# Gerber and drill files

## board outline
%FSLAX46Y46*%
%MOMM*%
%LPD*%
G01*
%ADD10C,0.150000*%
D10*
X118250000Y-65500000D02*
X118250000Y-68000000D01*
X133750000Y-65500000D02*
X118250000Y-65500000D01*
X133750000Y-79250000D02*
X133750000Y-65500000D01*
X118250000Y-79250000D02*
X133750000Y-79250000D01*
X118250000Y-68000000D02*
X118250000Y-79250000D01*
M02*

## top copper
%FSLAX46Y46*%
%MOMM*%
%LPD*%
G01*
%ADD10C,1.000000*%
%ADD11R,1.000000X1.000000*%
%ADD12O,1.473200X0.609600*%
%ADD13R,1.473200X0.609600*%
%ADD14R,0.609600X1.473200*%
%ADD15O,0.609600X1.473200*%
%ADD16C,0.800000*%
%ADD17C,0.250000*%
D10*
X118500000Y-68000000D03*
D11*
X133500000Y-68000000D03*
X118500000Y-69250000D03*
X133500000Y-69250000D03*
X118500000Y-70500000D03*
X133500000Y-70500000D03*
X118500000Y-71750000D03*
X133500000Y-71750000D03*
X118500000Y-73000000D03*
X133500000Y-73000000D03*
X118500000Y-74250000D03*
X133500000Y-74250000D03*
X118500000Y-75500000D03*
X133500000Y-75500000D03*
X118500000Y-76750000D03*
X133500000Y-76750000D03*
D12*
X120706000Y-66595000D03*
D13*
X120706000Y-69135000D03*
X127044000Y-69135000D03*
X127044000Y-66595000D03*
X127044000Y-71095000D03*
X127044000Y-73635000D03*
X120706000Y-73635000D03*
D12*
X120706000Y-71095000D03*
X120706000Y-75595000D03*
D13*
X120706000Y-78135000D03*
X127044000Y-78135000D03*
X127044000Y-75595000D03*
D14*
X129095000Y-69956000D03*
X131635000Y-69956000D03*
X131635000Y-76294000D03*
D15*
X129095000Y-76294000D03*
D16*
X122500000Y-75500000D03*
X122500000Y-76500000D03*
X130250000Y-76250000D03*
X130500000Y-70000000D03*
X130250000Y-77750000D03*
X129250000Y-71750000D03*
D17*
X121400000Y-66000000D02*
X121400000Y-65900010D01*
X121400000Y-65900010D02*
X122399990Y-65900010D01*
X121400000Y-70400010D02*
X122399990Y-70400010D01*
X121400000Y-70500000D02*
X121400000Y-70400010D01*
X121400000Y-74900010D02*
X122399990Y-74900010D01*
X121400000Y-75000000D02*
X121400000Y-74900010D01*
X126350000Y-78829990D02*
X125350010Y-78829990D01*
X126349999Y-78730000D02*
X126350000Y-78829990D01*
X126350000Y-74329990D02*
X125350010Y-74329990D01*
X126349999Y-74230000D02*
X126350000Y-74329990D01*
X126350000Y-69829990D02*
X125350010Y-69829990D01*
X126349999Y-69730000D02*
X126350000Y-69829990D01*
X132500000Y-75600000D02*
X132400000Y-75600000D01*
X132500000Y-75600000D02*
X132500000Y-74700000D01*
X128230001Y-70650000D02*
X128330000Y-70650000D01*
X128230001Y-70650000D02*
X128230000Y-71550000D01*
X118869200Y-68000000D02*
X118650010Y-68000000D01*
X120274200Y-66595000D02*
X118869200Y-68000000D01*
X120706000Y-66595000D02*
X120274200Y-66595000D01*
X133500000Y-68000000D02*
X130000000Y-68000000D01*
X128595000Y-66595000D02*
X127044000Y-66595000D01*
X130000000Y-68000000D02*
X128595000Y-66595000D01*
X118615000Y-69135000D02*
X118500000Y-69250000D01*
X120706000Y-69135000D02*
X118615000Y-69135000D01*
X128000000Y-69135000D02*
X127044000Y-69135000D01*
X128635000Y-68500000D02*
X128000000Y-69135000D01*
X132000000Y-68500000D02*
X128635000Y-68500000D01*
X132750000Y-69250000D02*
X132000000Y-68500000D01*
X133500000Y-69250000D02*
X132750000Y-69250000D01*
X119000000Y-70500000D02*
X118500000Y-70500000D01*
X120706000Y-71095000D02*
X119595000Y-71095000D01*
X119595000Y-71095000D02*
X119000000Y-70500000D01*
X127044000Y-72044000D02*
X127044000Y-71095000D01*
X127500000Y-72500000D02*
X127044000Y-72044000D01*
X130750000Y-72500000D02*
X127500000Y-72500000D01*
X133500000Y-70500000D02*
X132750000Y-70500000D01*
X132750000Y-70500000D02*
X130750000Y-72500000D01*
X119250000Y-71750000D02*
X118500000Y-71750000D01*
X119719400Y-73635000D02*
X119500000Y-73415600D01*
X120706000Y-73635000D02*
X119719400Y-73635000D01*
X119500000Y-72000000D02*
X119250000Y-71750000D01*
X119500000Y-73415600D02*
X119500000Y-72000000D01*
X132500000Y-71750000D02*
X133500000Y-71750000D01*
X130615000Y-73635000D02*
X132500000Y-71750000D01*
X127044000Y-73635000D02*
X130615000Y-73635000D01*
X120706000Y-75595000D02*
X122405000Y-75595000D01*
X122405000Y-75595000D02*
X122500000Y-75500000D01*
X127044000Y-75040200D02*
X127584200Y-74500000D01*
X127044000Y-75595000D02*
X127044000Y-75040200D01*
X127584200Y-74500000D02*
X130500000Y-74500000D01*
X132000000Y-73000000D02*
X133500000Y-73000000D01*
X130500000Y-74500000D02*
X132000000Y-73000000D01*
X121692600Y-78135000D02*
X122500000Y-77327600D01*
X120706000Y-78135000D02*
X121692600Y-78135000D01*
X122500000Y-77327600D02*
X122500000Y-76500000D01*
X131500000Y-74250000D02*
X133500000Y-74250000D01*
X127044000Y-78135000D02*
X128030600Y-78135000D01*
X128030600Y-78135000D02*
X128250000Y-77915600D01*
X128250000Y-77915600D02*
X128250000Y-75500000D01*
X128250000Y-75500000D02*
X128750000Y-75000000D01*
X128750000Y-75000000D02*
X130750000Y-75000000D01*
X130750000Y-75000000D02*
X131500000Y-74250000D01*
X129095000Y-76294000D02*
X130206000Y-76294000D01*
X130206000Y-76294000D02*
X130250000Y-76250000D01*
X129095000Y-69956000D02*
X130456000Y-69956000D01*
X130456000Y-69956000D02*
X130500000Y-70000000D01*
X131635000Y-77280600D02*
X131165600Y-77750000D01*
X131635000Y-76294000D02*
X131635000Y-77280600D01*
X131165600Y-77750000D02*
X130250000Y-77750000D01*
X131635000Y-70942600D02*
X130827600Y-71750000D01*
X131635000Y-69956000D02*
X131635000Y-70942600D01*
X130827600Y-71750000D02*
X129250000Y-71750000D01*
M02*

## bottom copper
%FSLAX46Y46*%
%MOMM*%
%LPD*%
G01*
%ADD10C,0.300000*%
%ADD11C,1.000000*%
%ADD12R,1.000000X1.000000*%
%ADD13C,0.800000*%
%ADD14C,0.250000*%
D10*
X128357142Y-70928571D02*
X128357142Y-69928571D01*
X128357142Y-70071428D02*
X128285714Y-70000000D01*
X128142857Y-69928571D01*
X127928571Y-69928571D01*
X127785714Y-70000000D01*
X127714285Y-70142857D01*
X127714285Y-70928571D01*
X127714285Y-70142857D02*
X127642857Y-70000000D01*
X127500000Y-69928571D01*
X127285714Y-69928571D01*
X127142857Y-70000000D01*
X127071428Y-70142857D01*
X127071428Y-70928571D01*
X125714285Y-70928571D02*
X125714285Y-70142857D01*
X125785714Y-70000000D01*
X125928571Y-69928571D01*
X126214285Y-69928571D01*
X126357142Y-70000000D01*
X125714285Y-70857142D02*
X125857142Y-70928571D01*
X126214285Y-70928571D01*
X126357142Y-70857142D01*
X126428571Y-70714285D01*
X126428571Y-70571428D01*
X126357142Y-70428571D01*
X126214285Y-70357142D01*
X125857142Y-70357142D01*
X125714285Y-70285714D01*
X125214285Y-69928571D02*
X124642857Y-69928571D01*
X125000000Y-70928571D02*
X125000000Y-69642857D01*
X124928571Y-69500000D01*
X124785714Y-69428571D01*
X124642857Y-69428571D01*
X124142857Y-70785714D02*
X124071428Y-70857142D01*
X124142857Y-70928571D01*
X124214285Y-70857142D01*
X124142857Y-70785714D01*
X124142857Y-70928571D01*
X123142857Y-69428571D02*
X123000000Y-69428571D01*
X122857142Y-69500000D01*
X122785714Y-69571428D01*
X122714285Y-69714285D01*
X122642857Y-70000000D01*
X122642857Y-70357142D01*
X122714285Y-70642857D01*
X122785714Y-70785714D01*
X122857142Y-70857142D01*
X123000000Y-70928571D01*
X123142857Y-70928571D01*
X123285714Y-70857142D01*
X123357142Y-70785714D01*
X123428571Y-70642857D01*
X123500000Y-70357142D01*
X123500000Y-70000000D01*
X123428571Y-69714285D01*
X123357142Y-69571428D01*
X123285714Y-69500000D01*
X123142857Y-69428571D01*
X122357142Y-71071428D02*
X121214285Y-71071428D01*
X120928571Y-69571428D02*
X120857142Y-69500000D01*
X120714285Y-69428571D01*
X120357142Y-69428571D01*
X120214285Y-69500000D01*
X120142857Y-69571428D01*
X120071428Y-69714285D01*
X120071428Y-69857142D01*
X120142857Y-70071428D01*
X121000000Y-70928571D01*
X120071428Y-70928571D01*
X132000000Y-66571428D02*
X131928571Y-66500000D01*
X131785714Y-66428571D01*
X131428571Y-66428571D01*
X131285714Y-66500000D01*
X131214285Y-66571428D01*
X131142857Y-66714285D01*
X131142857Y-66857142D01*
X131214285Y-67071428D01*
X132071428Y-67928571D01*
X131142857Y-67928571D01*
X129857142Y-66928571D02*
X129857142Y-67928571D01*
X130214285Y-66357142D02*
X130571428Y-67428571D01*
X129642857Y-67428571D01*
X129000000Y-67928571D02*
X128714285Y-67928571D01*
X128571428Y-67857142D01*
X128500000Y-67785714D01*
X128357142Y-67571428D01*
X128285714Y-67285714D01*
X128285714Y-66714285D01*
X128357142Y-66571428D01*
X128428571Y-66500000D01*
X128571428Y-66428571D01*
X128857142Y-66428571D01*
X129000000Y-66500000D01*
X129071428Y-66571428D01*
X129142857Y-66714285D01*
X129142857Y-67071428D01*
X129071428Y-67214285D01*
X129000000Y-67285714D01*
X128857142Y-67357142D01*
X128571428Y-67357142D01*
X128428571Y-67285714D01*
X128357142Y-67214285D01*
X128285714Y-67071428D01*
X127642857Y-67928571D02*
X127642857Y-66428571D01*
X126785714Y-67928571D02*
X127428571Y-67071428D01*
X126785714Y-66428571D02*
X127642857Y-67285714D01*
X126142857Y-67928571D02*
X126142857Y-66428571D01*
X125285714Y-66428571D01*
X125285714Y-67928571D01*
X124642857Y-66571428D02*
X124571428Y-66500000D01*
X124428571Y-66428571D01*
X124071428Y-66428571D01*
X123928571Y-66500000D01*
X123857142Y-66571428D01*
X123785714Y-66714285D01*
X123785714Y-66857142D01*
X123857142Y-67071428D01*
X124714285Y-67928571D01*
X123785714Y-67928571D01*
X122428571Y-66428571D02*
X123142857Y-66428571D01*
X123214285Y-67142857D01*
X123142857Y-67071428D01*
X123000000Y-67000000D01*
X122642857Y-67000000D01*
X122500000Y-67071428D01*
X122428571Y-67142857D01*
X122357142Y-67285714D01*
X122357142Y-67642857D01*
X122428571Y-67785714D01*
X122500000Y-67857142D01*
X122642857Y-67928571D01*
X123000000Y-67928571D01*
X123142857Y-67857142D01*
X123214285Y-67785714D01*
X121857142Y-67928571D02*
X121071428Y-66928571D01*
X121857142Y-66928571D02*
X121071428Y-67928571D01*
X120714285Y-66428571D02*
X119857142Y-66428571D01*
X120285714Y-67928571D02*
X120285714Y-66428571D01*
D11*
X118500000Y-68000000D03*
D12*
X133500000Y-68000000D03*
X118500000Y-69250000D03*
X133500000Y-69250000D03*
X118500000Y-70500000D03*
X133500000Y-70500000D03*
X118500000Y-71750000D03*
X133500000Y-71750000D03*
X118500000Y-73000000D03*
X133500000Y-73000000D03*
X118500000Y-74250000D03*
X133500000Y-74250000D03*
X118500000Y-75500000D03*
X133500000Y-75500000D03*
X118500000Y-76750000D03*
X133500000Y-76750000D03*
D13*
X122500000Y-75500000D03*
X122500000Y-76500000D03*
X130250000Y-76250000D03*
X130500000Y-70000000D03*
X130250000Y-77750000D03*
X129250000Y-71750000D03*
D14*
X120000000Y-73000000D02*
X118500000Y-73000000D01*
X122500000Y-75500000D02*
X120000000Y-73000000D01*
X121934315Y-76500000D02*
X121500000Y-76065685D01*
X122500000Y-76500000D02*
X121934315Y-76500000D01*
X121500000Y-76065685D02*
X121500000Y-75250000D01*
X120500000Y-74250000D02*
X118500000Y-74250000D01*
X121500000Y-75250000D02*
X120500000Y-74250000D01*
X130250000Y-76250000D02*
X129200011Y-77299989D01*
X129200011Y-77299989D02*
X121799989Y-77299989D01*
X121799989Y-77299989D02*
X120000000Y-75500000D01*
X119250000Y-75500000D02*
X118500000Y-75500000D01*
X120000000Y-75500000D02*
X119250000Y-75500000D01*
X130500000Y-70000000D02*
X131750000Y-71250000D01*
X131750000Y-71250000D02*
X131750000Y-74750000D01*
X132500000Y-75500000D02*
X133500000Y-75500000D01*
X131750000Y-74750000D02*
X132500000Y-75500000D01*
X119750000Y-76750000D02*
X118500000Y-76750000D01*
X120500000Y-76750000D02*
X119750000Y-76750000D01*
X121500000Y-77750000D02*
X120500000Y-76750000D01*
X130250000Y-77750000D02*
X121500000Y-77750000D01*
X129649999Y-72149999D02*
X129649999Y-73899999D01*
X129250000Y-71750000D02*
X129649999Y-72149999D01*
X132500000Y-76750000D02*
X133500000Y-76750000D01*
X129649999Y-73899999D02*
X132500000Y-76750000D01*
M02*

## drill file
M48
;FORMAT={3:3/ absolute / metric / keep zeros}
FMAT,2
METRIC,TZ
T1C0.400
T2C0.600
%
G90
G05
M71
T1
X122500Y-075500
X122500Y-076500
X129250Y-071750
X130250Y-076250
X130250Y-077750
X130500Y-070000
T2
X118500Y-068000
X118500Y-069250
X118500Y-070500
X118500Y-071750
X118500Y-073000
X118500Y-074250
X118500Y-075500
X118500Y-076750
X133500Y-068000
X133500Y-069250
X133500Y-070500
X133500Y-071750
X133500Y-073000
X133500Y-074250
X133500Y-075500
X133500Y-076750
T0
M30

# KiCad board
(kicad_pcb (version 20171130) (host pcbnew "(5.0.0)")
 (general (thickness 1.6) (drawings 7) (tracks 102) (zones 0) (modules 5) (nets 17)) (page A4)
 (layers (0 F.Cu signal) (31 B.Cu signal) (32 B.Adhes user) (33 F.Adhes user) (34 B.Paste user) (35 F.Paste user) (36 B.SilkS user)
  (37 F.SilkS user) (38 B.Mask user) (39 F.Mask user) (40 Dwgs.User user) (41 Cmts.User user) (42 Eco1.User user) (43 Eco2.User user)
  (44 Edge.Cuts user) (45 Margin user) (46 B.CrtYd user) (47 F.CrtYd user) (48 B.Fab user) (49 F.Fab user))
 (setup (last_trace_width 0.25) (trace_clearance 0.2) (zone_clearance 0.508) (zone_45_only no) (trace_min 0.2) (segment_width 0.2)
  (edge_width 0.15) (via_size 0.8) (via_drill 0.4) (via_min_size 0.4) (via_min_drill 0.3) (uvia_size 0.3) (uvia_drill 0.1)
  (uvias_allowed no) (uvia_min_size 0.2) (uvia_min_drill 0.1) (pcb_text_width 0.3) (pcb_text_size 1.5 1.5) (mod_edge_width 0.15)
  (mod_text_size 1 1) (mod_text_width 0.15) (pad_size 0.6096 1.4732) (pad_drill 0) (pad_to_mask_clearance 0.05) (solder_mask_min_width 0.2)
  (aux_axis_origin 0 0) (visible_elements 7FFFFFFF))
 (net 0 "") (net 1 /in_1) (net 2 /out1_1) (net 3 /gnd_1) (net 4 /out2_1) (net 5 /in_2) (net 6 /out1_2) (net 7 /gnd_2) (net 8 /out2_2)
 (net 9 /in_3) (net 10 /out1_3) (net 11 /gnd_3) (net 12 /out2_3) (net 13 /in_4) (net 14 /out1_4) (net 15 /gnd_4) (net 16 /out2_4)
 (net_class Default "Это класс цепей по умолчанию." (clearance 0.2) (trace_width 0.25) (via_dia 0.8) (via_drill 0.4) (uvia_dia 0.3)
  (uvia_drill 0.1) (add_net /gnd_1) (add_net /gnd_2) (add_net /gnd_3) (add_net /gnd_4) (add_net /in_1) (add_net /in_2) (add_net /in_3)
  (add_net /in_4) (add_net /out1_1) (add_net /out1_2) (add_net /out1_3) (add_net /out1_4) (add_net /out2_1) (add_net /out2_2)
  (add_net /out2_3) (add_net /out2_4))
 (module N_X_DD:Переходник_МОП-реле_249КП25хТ (layer F.Cu) (at 122 67)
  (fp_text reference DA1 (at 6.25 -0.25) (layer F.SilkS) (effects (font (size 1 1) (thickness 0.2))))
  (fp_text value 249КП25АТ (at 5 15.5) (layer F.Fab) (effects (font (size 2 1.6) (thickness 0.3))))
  (pad 1 thru_hole circle (at -3.5 1) (size 1 1) (drill 0.6) (layers *.Cu *.Mask) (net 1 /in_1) (clearance 0.2))
  (pad 16 thru_hole rect (at 11.5 1) (size 1 1) (drill 0.6) (layers *.Cu *.Mask) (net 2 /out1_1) (clearance 0.2))
  (pad 2 thru_hole rect (at -3.5 2.25) (size 1 1) (drill 0.6) (layers *.Cu *.Mask) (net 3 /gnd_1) (clearance 0.2))
  (pad 15 thru_hole rect (at 11.5 2.25) (size 1 1) (drill 0.6) (layers *.Cu *.Mask) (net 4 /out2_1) (clearance 0.2))
  (pad 3 thru_hole rect (at -3.5 3.5) (size 1 1) (drill 0.6) (layers *.Cu *.Mask) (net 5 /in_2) (clearance 0.2))
  (pad 14 thru_hole rect (at 11.5 3.5) (size 1 1) (drill 0.6) (layers *.Cu *.Mask) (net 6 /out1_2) (clearance 0.2))
  (pad 4 thru_hole rect (at -3.5 4.75) (size 1 1) (drill 0.6) (layers *.Cu *.Mask) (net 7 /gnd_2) (clearance 0.2))
  (pad 13 thru_hole rect (at 11.5 4.75) (size 1 1) (drill 0.6) (layers *.Cu *.Mask) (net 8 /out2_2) (clearance 0.2))
  (pad 5 thru_hole rect (at -3.5 6) (size 1 1) (drill 0.6) (layers *.Cu *.Mask) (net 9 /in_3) (clearance 0.2))
  (pad 12 thru_hole rect (at 11.5 6) (size 1 1) (drill 0.6) (layers *.Cu *.Mask) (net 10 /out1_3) (clearance 0.2))
  (pad 6 thru_hole rect (at -3.5 7.25) (size 1 1) (drill 0.6) (layers *.Cu *.Mask) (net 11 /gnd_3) (clearance 0.2))
  (pad 11 thru_hole rect (at 11.5 7.25) (size 1 1) (drill 0.6) (layers *.Cu *.Mask) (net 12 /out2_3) (clearance 0.2))
  (pad 7 thru_hole rect (at -3.5 8.5) (size 1 1) (drill 0.6) (layers *.Cu *.Mask) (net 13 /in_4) (clearance 0.2))
  (pad 10 thru_hole rect (at 11.5 8.5) (size 1 1) (drill 0.6) (layers *.Cu *.Mask) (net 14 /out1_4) (clearance 0.2))
  (pad 8 thru_hole rect (at -3.5 9.75) (size 1 1) (drill 0.6) (layers *.Cu *.Mask) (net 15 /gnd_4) (clearance 0.2))
  (pad 9 thru_hole rect (at 11.5 9.75) (size 1 1) (drill 0.6) (layers *.Cu *.Mask) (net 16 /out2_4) (clearance 0.2)))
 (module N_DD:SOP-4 (layer F.Cu) (at 123.5 68.5 270)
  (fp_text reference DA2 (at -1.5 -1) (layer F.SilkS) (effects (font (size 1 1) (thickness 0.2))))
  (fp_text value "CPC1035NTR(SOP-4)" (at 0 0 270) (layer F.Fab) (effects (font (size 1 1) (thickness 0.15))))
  (pad 1 smd oval (at -1.905 2.794 270) (size 0.6096 1.4732) (layers F.Cu F.Paste F.Mask) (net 1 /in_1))
  (pad 2 smd rect (at 0.635 2.794 270) (size 0.6096 1.4732) (layers F.Cu F.Paste F.Mask) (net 3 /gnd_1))
  (pad 3 smd rect (at 0.635 -3.544 270) (size 0.6096 1.4732) (layers F.Cu F.Paste F.Mask) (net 4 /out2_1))
  (pad 4 smd rect (at -1.905 -3.544 270) (size 0.6096 1.4732) (layers F.Cu F.Paste F.Mask) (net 2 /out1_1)))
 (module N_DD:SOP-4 (layer F.Cu) (at 123.5 73 270)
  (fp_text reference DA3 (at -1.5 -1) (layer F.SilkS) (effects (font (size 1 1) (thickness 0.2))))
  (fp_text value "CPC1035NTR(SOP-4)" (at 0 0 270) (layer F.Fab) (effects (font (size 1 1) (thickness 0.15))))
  (pad 4 smd rect (at -1.905 -3.544 270) (size 0.6096 1.4732) (layers F.Cu F.Paste F.Mask) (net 6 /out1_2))
  (pad 3 smd rect (at 0.635 -3.544 270) (size 0.6096 1.4732) (layers F.Cu F.Paste F.Mask) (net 8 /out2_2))
  (pad 2 smd rect (at 0.635 2.794 270) (size 0.6096 1.4732) (layers F.Cu F.Paste F.Mask) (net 7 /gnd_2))
  (pad 1 smd oval (at -1.905 2.794 270) (size 0.6096 1.4732) (layers F.Cu F.Paste F.Mask) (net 5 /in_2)))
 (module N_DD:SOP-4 (layer F.Cu) (at 123.5 77.5 270)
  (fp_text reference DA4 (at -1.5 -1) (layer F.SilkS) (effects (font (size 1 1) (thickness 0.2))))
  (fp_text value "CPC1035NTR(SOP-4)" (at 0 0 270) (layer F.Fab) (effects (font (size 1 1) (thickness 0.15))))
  (pad 1 smd oval (at -1.905 2.794 270) (size 0.6096 1.4732) (layers F.Cu F.Paste F.Mask) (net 9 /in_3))
  (pad 2 smd rect (at 0.635 2.794 270) (size 0.6096 1.4732) (layers F.Cu F.Paste F.Mask) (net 11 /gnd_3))
  (pad 3 smd rect (at 0.635 -3.544 270) (size 0.6096 1.4732) (layers F.Cu F.Paste F.Mask) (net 12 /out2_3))
  (pad 4 smd rect (at -1.905 -3.544 270) (size 0.6096 1.4732) (layers F.Cu F.Paste F.Mask) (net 10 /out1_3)))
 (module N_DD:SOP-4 (layer F.Cu) (at 131 73.5)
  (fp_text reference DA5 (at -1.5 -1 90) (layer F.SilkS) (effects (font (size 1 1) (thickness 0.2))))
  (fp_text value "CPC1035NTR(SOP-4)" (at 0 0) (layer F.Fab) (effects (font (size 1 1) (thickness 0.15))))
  (pad 4 smd rect (at -1.905 -3.544) (size 0.6096 1.4732) (layers F.Cu F.Paste F.Mask) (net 14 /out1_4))
  (pad 3 smd rect (at 0.635 -3.544) (size 0.6096 1.4732) (layers F.Cu F.Paste F.Mask) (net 16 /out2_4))
  (pad 2 smd rect (at 0.635 2.794) (size 0.6096 1.4732) (layers F.Cu F.Paste F.Mask) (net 15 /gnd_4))
  (pad 1 smd oval (at -1.905 2.794) (size 0.6096 1.4732) (layers F.Cu F.Paste F.Mask) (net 13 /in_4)))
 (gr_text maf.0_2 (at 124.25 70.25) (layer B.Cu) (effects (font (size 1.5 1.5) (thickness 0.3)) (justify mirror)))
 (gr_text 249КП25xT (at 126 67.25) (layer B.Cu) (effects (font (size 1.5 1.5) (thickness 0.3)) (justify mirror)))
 (gr_line (start 118.25 65.5) (end 118.25 68) (layer Edge.Cuts) (width 0.15))
 (gr_line (start 133.75 65.5) (end 118.25 65.5) (layer Edge.Cuts) (width 0.15))
 (gr_line (start 133.75 79.25) (end 133.75 65.5) (layer Edge.Cuts) (width 0.15))
 (gr_line (start 118.25 79.25) (end 133.75 79.25) (layer Edge.Cuts) (width 0.15))
 (gr_line (start 118.25 68) (end 118.25 79.25) (layer Edge.Cuts) (width 0.15))
 (segment (start 121.4 66) (end 121.4 65.90001) (width 0.25) (layer F.Cu) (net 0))
 (segment (start 121.4 65.90001) (end 122.39999 65.90001) (width 0.25) (layer F.Cu) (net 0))
 (segment (start 121.4 70.40001) (end 122.39999 70.40001) (width 0.25) (layer F.Cu) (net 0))
 (segment (start 121.4 70.5) (end 121.4 70.40001) (width 0.25) (layer F.Cu) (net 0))
 (segment (start 121.4 74.90001) (end 122.39999 74.90001) (width 0.25) (layer F.Cu) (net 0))
 (segment (start 121.4 75) (end 121.4 74.90001) (width 0.25) (layer F.Cu) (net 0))
 (segment (start 126.35 78.82999) (end 125.35001 78.82999) (width 0.25) (layer F.Cu) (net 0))
 (segment (start 126.349999 78.73) (end 126.35 78.82999) (width 0.25) (layer F.Cu) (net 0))
 (segment (start 126.35 74.32999) (end 125.35001 74.32999) (width 0.25) (layer F.Cu) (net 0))
 (segment (start 126.349999 74.23) (end 126.35 74.32999) (width 0.25) (layer F.Cu) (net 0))
 (segment (start 126.35 69.82999) (end 125.35001 69.82999) (width 0.25) (layer F.Cu) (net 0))
 (segment (start 126.349999 69.73) (end 126.35 69.82999) (width 0.25) (layer F.Cu) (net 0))
 (segment (start 132.5 75.6) (end 132.4 75.6) (width 0.25) (layer F.Cu) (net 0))
 (segment (start 132.5 75.6) (end 132.5 74.7) (width 0.25) (layer F.Cu) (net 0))
 (segment (start 128.230001 70.65) (end 128.33 70.65) (width 0.25) (layer F.Cu) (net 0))
 (segment (start 128.230001 70.65) (end 128.23 71.55) (width 0.25) (layer F.Cu) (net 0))
 (segment (start 118.8692 68) (end 118.65001 68) (width 0.25) (layer F.Cu) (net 1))
 (segment (start 120.2742 66.595) (end 118.8692 68) (width 0.25) (layer F.Cu) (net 1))
 (segment (start 120.706 66.595) (end 120.2742 66.595) (width 0.25) (layer F.Cu) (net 1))
 (segment (start 133.5 68) (end 130 68) (width 0.25) (layer F.Cu) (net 2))
 (segment (start 128.595 66.595) (end 127.044 66.595) (width 0.25) (layer F.Cu) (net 2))
 (segment (start 130 68) (end 128.595 66.595) (width 0.25) (layer F.Cu) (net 2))
 (segment (start 118.615 69.135) (end 118.5 69.25) (width 0.25) (layer F.Cu) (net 3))
 (segment (start 120.706 69.135) (end 118.615 69.135) (width 0.25) (layer F.Cu) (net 3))
 (segment (start 128 69.135) (end 127.044 69.135) (width 0.25) (layer F.Cu) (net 4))
 (segment (start 128.635 68.5) (end 128 69.135) (width 0.25) (layer F.Cu) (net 4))
 (segment (start 132 68.5) (end 128.635 68.5) (width 0.25) (layer F.Cu) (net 4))
 (segment (start 132.75 69.25) (end 132 68.5) (width 0.25) (layer F.Cu) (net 4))
 (segment (start 133.5 69.25) (end 132.75 69.25) (width 0.25) (layer F.Cu) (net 4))
 (segment (start 119 70.5) (end 118.5 70.5) (width 0.25) (layer F.Cu) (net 5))
 (segment (start 120.706 71.095) (end 119.595 71.095) (width 0.25) (layer F.Cu) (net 5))
 (segment (start 119.595 71.095) (end 119 70.5) (width 0.25) (layer F.Cu) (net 5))
 (segment (start 127.044 72.044) (end 127.044 71.095) (width 0.25) (layer F.Cu) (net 6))
 (segment (start 127.5 72.5) (end 127.044 72.044) (width 0.25) (layer F.Cu) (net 6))
 (segment (start 130.75 72.5) (end 127.5 72.5) (width 0.25) (layer F.Cu) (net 6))
 (segment (start 133.5 70.5) (end 132.75 70.5) (width 0.25) (layer F.Cu) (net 6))
 (segment (start 132.75 70.5) (end 130.75 72.5) (width 0.25) (layer F.Cu) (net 6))
 (segment (start 119.25 71.75) (end 118.5 71.75) (width 0.25) (layer F.Cu) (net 7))
 (segment (start 119.7194 73.635) (end 119.5 73.4156) (width 0.25) (layer F.Cu) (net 7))
 (segment (start 120.706 73.635) (end 119.7194 73.635) (width 0.25) (layer F.Cu) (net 7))
 (segment (start 119.5 72) (end 119.25 71.75) (width 0.25) (layer F.Cu) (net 7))
 (segment (start 119.5 73.4156) (end 119.5 72) (width 0.25) (layer F.Cu) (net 7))
 (segment (start 132.5 71.75) (end 133.5 71.75) (width 0.25) (layer F.Cu) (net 8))
 (segment (start 130.615 73.635) (end 132.5 71.75) (width 0.25) (layer F.Cu) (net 8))
 (segment (start 127.044 73.635) (end 130.615 73.635) (width 0.25) (layer F.Cu) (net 8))
 (via (at 122.5 75.5) (size 0.8) (drill 0.4) (layers F.Cu B.Cu) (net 9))
 (segment (start 120.706 75.595) (end 122.405 75.595) (width 0.25) (layer F.Cu) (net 9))
 (segment (start 122.405 75.595) (end 122.5 75.5) (width 0.25) (layer F.Cu) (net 9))
 (segment (start 120 73) (end 118.5 73) (width 0.25) (layer B.Cu) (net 9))
 (segment (start 122.5 75.5) (end 120 73) (width 0.25) (layer B.Cu) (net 9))
 (segment (start 127.044 75.0402) (end 127.5842 74.5) (width 0.25) (layer F.Cu) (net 10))
 (segment (start 127.044 75.595) (end 127.044 75.0402) (width 0.25) (layer F.Cu) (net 10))
 (segment (start 127.5842 74.5) (end 130.5 74.5) (width 0.25) (layer F.Cu) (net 10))
 (segment (start 132 73) (end 133.5 73) (width 0.25) (layer F.Cu) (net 10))
 (segment (start 130.5 74.5) (end 132 73) (width 0.25) (layer F.Cu) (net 10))
 (via (at 122.5 76.5) (size 0.8) (drill 0.4) (layers F.Cu B.Cu) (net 11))
 (segment (start 121.934315 76.5) (end 121.5 76.065685) (width 0.25) (layer B.Cu) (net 11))
 (segment (start 122.5 76.5) (end 121.934315 76.5) (width 0.25) (layer B.Cu) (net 11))
 (segment (start 121.5 76.065685) (end 121.5 75.25) (width 0.25) (layer B.Cu) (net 11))
 (segment (start 120.5 74.25) (end 118.5 74.25) (width 0.25) (layer B.Cu) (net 11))
 (segment (start 121.5 75.25) (end 120.5 74.25) (width 0.25) (layer B.Cu) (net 11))
 (segment (start 121.6926 78.135) (end 122.5 77.3276) (width 0.25) (layer F.Cu) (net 11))
 (segment (start 120.706 78.135) (end 121.6926 78.135) (width 0.25) (layer F.Cu) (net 11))
 (segment (start 122.5 77.3276) (end 122.5 76.5) (width 0.25) (layer F.Cu) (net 11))
 (segment (start 131.5 74.25) (end 133.5 74.25) (width 0.25) (layer F.Cu) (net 12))
 (segment (start 127.044 78.135) (end 128.0306 78.135) (width 0.25) (layer F.Cu) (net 12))
 (segment (start 128.0306 78.135) (end 128.25 77.9156) (width 0.25) (layer F.Cu) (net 12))
 (segment (start 128.25 77.9156) (end 128.25 75.5) (width 0.25) (layer F.Cu) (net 12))
 (segment (start 128.25 75.5) (end 128.75 75) (width 0.25) (layer F.Cu) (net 12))
 (segment (start 128.75 75) (end 130.75 75) (width 0.25) (layer F.Cu) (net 12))
 (segment (start 130.75 75) (end 131.5 74.25) (width 0.25) (layer F.Cu) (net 12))
 (via (at 130.25 76.25) (size 0.8) (drill 0.4) (layers F.Cu B.Cu) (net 13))
 (segment (start 129.095 76.294) (end 130.206 76.294) (width 0.25) (layer F.Cu) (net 13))
 (segment (start 130.206 76.294) (end 130.25 76.25) (width 0.25) (layer F.Cu) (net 13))
 (segment (start 130.25 76.25) (end 129.200011 77.299989) (width 0.25) (layer B.Cu) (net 13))
 (segment (start 129.200011 77.299989) (end 121.799989 77.299989) (width 0.25) (layer B.Cu) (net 13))
 (segment (start 121.799989 77.299989) (end 120 75.5) (width 0.25) (layer B.Cu) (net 13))
 (segment (start 119.25 75.5) (end 118.5 75.5) (width 0.25) (layer B.Cu) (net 13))
 (segment (start 120 75.5) (end 119.25 75.5) (width 0.25) (layer B.Cu) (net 13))
 (via (at 130.5 70) (size 0.8) (drill 0.4) (layers F.Cu B.Cu) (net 14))
 (segment (start 129.095 69.956) (end 130.456 69.956) (width 0.25) (layer F.Cu) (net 14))
 (segment (start 130.456 69.956) (end 130.5 70) (width 0.25) (layer F.Cu) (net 14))
 (segment (start 130.5 70) (end 131.75 71.25) (width 0.25) (layer B.Cu) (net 14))
 (segment (start 131.75 71.25) (end 131.75 74.75) (width 0.25) (layer B.Cu) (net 14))
 (segment (start 132.5 75.5) (end 133.5 75.5) (width 0.25) (layer B.Cu) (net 14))
 (segment (start 131.75 74.75) (end 132.5 75.5) (width 0.25) (layer B.Cu) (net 14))
 (via (at 130.25 77.75) (size 0.8) (drill 0.4) (layers F.Cu B.Cu) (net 15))
 (segment (start 119.75 76.75) (end 118.5 76.75) (width 0.25) (layer B.Cu) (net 15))
 (segment (start 120.5 76.75) (end 119.75 76.75) (width 0.25) (layer B.Cu) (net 15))
 (segment (start 121.5 77.75) (end 120.5 76.75) (width 0.25) (layer B.Cu) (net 15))
 (segment (start 130.25 77.75) (end 121.5 77.75) (width 0.25) (layer B.Cu) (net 15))
 (segment (start 131.635 77.2806) (end 131.1656 77.75) (width 0.25) (layer F.Cu) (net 15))
 (segment (start 131.635 76.294) (end 131.635 77.2806) (width 0.25) (layer F.Cu) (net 15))
 (segment (start 131.1656 77.75) (end 130.25 77.75) (width 0.25) (layer F.Cu) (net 15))
 (via (at 129.25 71.75) (size 0.8) (drill 0.4) (layers F.Cu B.Cu) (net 16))
 (segment (start 131.635 70.9426) (end 130.8276 71.75) (width 0.25) (layer F.Cu) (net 16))
 (segment (start 131.635 69.956) (end 131.635 70.9426) (width 0.25) (layer F.Cu) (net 16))
 (segment (start 130.8276 71.75) (end 129.25 71.75) (width 0.25) (layer F.Cu) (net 16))
 (segment (start 129.649999 72.149999) (end 129.649999 73.899999) (width 0.25) (layer B.Cu) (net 16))
 (segment (start 129.25 71.75) (end 129.649999 72.149999) (width 0.25) (layer B.Cu) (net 16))
 (segment (start 132.5 76.75) (end 133.5 76.75) (width 0.25) (layer B.Cu) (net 16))
 (segment (start 129.649999 73.899999) (end 132.5 76.75) (width 0.25) (layer B.Cu) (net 16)))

